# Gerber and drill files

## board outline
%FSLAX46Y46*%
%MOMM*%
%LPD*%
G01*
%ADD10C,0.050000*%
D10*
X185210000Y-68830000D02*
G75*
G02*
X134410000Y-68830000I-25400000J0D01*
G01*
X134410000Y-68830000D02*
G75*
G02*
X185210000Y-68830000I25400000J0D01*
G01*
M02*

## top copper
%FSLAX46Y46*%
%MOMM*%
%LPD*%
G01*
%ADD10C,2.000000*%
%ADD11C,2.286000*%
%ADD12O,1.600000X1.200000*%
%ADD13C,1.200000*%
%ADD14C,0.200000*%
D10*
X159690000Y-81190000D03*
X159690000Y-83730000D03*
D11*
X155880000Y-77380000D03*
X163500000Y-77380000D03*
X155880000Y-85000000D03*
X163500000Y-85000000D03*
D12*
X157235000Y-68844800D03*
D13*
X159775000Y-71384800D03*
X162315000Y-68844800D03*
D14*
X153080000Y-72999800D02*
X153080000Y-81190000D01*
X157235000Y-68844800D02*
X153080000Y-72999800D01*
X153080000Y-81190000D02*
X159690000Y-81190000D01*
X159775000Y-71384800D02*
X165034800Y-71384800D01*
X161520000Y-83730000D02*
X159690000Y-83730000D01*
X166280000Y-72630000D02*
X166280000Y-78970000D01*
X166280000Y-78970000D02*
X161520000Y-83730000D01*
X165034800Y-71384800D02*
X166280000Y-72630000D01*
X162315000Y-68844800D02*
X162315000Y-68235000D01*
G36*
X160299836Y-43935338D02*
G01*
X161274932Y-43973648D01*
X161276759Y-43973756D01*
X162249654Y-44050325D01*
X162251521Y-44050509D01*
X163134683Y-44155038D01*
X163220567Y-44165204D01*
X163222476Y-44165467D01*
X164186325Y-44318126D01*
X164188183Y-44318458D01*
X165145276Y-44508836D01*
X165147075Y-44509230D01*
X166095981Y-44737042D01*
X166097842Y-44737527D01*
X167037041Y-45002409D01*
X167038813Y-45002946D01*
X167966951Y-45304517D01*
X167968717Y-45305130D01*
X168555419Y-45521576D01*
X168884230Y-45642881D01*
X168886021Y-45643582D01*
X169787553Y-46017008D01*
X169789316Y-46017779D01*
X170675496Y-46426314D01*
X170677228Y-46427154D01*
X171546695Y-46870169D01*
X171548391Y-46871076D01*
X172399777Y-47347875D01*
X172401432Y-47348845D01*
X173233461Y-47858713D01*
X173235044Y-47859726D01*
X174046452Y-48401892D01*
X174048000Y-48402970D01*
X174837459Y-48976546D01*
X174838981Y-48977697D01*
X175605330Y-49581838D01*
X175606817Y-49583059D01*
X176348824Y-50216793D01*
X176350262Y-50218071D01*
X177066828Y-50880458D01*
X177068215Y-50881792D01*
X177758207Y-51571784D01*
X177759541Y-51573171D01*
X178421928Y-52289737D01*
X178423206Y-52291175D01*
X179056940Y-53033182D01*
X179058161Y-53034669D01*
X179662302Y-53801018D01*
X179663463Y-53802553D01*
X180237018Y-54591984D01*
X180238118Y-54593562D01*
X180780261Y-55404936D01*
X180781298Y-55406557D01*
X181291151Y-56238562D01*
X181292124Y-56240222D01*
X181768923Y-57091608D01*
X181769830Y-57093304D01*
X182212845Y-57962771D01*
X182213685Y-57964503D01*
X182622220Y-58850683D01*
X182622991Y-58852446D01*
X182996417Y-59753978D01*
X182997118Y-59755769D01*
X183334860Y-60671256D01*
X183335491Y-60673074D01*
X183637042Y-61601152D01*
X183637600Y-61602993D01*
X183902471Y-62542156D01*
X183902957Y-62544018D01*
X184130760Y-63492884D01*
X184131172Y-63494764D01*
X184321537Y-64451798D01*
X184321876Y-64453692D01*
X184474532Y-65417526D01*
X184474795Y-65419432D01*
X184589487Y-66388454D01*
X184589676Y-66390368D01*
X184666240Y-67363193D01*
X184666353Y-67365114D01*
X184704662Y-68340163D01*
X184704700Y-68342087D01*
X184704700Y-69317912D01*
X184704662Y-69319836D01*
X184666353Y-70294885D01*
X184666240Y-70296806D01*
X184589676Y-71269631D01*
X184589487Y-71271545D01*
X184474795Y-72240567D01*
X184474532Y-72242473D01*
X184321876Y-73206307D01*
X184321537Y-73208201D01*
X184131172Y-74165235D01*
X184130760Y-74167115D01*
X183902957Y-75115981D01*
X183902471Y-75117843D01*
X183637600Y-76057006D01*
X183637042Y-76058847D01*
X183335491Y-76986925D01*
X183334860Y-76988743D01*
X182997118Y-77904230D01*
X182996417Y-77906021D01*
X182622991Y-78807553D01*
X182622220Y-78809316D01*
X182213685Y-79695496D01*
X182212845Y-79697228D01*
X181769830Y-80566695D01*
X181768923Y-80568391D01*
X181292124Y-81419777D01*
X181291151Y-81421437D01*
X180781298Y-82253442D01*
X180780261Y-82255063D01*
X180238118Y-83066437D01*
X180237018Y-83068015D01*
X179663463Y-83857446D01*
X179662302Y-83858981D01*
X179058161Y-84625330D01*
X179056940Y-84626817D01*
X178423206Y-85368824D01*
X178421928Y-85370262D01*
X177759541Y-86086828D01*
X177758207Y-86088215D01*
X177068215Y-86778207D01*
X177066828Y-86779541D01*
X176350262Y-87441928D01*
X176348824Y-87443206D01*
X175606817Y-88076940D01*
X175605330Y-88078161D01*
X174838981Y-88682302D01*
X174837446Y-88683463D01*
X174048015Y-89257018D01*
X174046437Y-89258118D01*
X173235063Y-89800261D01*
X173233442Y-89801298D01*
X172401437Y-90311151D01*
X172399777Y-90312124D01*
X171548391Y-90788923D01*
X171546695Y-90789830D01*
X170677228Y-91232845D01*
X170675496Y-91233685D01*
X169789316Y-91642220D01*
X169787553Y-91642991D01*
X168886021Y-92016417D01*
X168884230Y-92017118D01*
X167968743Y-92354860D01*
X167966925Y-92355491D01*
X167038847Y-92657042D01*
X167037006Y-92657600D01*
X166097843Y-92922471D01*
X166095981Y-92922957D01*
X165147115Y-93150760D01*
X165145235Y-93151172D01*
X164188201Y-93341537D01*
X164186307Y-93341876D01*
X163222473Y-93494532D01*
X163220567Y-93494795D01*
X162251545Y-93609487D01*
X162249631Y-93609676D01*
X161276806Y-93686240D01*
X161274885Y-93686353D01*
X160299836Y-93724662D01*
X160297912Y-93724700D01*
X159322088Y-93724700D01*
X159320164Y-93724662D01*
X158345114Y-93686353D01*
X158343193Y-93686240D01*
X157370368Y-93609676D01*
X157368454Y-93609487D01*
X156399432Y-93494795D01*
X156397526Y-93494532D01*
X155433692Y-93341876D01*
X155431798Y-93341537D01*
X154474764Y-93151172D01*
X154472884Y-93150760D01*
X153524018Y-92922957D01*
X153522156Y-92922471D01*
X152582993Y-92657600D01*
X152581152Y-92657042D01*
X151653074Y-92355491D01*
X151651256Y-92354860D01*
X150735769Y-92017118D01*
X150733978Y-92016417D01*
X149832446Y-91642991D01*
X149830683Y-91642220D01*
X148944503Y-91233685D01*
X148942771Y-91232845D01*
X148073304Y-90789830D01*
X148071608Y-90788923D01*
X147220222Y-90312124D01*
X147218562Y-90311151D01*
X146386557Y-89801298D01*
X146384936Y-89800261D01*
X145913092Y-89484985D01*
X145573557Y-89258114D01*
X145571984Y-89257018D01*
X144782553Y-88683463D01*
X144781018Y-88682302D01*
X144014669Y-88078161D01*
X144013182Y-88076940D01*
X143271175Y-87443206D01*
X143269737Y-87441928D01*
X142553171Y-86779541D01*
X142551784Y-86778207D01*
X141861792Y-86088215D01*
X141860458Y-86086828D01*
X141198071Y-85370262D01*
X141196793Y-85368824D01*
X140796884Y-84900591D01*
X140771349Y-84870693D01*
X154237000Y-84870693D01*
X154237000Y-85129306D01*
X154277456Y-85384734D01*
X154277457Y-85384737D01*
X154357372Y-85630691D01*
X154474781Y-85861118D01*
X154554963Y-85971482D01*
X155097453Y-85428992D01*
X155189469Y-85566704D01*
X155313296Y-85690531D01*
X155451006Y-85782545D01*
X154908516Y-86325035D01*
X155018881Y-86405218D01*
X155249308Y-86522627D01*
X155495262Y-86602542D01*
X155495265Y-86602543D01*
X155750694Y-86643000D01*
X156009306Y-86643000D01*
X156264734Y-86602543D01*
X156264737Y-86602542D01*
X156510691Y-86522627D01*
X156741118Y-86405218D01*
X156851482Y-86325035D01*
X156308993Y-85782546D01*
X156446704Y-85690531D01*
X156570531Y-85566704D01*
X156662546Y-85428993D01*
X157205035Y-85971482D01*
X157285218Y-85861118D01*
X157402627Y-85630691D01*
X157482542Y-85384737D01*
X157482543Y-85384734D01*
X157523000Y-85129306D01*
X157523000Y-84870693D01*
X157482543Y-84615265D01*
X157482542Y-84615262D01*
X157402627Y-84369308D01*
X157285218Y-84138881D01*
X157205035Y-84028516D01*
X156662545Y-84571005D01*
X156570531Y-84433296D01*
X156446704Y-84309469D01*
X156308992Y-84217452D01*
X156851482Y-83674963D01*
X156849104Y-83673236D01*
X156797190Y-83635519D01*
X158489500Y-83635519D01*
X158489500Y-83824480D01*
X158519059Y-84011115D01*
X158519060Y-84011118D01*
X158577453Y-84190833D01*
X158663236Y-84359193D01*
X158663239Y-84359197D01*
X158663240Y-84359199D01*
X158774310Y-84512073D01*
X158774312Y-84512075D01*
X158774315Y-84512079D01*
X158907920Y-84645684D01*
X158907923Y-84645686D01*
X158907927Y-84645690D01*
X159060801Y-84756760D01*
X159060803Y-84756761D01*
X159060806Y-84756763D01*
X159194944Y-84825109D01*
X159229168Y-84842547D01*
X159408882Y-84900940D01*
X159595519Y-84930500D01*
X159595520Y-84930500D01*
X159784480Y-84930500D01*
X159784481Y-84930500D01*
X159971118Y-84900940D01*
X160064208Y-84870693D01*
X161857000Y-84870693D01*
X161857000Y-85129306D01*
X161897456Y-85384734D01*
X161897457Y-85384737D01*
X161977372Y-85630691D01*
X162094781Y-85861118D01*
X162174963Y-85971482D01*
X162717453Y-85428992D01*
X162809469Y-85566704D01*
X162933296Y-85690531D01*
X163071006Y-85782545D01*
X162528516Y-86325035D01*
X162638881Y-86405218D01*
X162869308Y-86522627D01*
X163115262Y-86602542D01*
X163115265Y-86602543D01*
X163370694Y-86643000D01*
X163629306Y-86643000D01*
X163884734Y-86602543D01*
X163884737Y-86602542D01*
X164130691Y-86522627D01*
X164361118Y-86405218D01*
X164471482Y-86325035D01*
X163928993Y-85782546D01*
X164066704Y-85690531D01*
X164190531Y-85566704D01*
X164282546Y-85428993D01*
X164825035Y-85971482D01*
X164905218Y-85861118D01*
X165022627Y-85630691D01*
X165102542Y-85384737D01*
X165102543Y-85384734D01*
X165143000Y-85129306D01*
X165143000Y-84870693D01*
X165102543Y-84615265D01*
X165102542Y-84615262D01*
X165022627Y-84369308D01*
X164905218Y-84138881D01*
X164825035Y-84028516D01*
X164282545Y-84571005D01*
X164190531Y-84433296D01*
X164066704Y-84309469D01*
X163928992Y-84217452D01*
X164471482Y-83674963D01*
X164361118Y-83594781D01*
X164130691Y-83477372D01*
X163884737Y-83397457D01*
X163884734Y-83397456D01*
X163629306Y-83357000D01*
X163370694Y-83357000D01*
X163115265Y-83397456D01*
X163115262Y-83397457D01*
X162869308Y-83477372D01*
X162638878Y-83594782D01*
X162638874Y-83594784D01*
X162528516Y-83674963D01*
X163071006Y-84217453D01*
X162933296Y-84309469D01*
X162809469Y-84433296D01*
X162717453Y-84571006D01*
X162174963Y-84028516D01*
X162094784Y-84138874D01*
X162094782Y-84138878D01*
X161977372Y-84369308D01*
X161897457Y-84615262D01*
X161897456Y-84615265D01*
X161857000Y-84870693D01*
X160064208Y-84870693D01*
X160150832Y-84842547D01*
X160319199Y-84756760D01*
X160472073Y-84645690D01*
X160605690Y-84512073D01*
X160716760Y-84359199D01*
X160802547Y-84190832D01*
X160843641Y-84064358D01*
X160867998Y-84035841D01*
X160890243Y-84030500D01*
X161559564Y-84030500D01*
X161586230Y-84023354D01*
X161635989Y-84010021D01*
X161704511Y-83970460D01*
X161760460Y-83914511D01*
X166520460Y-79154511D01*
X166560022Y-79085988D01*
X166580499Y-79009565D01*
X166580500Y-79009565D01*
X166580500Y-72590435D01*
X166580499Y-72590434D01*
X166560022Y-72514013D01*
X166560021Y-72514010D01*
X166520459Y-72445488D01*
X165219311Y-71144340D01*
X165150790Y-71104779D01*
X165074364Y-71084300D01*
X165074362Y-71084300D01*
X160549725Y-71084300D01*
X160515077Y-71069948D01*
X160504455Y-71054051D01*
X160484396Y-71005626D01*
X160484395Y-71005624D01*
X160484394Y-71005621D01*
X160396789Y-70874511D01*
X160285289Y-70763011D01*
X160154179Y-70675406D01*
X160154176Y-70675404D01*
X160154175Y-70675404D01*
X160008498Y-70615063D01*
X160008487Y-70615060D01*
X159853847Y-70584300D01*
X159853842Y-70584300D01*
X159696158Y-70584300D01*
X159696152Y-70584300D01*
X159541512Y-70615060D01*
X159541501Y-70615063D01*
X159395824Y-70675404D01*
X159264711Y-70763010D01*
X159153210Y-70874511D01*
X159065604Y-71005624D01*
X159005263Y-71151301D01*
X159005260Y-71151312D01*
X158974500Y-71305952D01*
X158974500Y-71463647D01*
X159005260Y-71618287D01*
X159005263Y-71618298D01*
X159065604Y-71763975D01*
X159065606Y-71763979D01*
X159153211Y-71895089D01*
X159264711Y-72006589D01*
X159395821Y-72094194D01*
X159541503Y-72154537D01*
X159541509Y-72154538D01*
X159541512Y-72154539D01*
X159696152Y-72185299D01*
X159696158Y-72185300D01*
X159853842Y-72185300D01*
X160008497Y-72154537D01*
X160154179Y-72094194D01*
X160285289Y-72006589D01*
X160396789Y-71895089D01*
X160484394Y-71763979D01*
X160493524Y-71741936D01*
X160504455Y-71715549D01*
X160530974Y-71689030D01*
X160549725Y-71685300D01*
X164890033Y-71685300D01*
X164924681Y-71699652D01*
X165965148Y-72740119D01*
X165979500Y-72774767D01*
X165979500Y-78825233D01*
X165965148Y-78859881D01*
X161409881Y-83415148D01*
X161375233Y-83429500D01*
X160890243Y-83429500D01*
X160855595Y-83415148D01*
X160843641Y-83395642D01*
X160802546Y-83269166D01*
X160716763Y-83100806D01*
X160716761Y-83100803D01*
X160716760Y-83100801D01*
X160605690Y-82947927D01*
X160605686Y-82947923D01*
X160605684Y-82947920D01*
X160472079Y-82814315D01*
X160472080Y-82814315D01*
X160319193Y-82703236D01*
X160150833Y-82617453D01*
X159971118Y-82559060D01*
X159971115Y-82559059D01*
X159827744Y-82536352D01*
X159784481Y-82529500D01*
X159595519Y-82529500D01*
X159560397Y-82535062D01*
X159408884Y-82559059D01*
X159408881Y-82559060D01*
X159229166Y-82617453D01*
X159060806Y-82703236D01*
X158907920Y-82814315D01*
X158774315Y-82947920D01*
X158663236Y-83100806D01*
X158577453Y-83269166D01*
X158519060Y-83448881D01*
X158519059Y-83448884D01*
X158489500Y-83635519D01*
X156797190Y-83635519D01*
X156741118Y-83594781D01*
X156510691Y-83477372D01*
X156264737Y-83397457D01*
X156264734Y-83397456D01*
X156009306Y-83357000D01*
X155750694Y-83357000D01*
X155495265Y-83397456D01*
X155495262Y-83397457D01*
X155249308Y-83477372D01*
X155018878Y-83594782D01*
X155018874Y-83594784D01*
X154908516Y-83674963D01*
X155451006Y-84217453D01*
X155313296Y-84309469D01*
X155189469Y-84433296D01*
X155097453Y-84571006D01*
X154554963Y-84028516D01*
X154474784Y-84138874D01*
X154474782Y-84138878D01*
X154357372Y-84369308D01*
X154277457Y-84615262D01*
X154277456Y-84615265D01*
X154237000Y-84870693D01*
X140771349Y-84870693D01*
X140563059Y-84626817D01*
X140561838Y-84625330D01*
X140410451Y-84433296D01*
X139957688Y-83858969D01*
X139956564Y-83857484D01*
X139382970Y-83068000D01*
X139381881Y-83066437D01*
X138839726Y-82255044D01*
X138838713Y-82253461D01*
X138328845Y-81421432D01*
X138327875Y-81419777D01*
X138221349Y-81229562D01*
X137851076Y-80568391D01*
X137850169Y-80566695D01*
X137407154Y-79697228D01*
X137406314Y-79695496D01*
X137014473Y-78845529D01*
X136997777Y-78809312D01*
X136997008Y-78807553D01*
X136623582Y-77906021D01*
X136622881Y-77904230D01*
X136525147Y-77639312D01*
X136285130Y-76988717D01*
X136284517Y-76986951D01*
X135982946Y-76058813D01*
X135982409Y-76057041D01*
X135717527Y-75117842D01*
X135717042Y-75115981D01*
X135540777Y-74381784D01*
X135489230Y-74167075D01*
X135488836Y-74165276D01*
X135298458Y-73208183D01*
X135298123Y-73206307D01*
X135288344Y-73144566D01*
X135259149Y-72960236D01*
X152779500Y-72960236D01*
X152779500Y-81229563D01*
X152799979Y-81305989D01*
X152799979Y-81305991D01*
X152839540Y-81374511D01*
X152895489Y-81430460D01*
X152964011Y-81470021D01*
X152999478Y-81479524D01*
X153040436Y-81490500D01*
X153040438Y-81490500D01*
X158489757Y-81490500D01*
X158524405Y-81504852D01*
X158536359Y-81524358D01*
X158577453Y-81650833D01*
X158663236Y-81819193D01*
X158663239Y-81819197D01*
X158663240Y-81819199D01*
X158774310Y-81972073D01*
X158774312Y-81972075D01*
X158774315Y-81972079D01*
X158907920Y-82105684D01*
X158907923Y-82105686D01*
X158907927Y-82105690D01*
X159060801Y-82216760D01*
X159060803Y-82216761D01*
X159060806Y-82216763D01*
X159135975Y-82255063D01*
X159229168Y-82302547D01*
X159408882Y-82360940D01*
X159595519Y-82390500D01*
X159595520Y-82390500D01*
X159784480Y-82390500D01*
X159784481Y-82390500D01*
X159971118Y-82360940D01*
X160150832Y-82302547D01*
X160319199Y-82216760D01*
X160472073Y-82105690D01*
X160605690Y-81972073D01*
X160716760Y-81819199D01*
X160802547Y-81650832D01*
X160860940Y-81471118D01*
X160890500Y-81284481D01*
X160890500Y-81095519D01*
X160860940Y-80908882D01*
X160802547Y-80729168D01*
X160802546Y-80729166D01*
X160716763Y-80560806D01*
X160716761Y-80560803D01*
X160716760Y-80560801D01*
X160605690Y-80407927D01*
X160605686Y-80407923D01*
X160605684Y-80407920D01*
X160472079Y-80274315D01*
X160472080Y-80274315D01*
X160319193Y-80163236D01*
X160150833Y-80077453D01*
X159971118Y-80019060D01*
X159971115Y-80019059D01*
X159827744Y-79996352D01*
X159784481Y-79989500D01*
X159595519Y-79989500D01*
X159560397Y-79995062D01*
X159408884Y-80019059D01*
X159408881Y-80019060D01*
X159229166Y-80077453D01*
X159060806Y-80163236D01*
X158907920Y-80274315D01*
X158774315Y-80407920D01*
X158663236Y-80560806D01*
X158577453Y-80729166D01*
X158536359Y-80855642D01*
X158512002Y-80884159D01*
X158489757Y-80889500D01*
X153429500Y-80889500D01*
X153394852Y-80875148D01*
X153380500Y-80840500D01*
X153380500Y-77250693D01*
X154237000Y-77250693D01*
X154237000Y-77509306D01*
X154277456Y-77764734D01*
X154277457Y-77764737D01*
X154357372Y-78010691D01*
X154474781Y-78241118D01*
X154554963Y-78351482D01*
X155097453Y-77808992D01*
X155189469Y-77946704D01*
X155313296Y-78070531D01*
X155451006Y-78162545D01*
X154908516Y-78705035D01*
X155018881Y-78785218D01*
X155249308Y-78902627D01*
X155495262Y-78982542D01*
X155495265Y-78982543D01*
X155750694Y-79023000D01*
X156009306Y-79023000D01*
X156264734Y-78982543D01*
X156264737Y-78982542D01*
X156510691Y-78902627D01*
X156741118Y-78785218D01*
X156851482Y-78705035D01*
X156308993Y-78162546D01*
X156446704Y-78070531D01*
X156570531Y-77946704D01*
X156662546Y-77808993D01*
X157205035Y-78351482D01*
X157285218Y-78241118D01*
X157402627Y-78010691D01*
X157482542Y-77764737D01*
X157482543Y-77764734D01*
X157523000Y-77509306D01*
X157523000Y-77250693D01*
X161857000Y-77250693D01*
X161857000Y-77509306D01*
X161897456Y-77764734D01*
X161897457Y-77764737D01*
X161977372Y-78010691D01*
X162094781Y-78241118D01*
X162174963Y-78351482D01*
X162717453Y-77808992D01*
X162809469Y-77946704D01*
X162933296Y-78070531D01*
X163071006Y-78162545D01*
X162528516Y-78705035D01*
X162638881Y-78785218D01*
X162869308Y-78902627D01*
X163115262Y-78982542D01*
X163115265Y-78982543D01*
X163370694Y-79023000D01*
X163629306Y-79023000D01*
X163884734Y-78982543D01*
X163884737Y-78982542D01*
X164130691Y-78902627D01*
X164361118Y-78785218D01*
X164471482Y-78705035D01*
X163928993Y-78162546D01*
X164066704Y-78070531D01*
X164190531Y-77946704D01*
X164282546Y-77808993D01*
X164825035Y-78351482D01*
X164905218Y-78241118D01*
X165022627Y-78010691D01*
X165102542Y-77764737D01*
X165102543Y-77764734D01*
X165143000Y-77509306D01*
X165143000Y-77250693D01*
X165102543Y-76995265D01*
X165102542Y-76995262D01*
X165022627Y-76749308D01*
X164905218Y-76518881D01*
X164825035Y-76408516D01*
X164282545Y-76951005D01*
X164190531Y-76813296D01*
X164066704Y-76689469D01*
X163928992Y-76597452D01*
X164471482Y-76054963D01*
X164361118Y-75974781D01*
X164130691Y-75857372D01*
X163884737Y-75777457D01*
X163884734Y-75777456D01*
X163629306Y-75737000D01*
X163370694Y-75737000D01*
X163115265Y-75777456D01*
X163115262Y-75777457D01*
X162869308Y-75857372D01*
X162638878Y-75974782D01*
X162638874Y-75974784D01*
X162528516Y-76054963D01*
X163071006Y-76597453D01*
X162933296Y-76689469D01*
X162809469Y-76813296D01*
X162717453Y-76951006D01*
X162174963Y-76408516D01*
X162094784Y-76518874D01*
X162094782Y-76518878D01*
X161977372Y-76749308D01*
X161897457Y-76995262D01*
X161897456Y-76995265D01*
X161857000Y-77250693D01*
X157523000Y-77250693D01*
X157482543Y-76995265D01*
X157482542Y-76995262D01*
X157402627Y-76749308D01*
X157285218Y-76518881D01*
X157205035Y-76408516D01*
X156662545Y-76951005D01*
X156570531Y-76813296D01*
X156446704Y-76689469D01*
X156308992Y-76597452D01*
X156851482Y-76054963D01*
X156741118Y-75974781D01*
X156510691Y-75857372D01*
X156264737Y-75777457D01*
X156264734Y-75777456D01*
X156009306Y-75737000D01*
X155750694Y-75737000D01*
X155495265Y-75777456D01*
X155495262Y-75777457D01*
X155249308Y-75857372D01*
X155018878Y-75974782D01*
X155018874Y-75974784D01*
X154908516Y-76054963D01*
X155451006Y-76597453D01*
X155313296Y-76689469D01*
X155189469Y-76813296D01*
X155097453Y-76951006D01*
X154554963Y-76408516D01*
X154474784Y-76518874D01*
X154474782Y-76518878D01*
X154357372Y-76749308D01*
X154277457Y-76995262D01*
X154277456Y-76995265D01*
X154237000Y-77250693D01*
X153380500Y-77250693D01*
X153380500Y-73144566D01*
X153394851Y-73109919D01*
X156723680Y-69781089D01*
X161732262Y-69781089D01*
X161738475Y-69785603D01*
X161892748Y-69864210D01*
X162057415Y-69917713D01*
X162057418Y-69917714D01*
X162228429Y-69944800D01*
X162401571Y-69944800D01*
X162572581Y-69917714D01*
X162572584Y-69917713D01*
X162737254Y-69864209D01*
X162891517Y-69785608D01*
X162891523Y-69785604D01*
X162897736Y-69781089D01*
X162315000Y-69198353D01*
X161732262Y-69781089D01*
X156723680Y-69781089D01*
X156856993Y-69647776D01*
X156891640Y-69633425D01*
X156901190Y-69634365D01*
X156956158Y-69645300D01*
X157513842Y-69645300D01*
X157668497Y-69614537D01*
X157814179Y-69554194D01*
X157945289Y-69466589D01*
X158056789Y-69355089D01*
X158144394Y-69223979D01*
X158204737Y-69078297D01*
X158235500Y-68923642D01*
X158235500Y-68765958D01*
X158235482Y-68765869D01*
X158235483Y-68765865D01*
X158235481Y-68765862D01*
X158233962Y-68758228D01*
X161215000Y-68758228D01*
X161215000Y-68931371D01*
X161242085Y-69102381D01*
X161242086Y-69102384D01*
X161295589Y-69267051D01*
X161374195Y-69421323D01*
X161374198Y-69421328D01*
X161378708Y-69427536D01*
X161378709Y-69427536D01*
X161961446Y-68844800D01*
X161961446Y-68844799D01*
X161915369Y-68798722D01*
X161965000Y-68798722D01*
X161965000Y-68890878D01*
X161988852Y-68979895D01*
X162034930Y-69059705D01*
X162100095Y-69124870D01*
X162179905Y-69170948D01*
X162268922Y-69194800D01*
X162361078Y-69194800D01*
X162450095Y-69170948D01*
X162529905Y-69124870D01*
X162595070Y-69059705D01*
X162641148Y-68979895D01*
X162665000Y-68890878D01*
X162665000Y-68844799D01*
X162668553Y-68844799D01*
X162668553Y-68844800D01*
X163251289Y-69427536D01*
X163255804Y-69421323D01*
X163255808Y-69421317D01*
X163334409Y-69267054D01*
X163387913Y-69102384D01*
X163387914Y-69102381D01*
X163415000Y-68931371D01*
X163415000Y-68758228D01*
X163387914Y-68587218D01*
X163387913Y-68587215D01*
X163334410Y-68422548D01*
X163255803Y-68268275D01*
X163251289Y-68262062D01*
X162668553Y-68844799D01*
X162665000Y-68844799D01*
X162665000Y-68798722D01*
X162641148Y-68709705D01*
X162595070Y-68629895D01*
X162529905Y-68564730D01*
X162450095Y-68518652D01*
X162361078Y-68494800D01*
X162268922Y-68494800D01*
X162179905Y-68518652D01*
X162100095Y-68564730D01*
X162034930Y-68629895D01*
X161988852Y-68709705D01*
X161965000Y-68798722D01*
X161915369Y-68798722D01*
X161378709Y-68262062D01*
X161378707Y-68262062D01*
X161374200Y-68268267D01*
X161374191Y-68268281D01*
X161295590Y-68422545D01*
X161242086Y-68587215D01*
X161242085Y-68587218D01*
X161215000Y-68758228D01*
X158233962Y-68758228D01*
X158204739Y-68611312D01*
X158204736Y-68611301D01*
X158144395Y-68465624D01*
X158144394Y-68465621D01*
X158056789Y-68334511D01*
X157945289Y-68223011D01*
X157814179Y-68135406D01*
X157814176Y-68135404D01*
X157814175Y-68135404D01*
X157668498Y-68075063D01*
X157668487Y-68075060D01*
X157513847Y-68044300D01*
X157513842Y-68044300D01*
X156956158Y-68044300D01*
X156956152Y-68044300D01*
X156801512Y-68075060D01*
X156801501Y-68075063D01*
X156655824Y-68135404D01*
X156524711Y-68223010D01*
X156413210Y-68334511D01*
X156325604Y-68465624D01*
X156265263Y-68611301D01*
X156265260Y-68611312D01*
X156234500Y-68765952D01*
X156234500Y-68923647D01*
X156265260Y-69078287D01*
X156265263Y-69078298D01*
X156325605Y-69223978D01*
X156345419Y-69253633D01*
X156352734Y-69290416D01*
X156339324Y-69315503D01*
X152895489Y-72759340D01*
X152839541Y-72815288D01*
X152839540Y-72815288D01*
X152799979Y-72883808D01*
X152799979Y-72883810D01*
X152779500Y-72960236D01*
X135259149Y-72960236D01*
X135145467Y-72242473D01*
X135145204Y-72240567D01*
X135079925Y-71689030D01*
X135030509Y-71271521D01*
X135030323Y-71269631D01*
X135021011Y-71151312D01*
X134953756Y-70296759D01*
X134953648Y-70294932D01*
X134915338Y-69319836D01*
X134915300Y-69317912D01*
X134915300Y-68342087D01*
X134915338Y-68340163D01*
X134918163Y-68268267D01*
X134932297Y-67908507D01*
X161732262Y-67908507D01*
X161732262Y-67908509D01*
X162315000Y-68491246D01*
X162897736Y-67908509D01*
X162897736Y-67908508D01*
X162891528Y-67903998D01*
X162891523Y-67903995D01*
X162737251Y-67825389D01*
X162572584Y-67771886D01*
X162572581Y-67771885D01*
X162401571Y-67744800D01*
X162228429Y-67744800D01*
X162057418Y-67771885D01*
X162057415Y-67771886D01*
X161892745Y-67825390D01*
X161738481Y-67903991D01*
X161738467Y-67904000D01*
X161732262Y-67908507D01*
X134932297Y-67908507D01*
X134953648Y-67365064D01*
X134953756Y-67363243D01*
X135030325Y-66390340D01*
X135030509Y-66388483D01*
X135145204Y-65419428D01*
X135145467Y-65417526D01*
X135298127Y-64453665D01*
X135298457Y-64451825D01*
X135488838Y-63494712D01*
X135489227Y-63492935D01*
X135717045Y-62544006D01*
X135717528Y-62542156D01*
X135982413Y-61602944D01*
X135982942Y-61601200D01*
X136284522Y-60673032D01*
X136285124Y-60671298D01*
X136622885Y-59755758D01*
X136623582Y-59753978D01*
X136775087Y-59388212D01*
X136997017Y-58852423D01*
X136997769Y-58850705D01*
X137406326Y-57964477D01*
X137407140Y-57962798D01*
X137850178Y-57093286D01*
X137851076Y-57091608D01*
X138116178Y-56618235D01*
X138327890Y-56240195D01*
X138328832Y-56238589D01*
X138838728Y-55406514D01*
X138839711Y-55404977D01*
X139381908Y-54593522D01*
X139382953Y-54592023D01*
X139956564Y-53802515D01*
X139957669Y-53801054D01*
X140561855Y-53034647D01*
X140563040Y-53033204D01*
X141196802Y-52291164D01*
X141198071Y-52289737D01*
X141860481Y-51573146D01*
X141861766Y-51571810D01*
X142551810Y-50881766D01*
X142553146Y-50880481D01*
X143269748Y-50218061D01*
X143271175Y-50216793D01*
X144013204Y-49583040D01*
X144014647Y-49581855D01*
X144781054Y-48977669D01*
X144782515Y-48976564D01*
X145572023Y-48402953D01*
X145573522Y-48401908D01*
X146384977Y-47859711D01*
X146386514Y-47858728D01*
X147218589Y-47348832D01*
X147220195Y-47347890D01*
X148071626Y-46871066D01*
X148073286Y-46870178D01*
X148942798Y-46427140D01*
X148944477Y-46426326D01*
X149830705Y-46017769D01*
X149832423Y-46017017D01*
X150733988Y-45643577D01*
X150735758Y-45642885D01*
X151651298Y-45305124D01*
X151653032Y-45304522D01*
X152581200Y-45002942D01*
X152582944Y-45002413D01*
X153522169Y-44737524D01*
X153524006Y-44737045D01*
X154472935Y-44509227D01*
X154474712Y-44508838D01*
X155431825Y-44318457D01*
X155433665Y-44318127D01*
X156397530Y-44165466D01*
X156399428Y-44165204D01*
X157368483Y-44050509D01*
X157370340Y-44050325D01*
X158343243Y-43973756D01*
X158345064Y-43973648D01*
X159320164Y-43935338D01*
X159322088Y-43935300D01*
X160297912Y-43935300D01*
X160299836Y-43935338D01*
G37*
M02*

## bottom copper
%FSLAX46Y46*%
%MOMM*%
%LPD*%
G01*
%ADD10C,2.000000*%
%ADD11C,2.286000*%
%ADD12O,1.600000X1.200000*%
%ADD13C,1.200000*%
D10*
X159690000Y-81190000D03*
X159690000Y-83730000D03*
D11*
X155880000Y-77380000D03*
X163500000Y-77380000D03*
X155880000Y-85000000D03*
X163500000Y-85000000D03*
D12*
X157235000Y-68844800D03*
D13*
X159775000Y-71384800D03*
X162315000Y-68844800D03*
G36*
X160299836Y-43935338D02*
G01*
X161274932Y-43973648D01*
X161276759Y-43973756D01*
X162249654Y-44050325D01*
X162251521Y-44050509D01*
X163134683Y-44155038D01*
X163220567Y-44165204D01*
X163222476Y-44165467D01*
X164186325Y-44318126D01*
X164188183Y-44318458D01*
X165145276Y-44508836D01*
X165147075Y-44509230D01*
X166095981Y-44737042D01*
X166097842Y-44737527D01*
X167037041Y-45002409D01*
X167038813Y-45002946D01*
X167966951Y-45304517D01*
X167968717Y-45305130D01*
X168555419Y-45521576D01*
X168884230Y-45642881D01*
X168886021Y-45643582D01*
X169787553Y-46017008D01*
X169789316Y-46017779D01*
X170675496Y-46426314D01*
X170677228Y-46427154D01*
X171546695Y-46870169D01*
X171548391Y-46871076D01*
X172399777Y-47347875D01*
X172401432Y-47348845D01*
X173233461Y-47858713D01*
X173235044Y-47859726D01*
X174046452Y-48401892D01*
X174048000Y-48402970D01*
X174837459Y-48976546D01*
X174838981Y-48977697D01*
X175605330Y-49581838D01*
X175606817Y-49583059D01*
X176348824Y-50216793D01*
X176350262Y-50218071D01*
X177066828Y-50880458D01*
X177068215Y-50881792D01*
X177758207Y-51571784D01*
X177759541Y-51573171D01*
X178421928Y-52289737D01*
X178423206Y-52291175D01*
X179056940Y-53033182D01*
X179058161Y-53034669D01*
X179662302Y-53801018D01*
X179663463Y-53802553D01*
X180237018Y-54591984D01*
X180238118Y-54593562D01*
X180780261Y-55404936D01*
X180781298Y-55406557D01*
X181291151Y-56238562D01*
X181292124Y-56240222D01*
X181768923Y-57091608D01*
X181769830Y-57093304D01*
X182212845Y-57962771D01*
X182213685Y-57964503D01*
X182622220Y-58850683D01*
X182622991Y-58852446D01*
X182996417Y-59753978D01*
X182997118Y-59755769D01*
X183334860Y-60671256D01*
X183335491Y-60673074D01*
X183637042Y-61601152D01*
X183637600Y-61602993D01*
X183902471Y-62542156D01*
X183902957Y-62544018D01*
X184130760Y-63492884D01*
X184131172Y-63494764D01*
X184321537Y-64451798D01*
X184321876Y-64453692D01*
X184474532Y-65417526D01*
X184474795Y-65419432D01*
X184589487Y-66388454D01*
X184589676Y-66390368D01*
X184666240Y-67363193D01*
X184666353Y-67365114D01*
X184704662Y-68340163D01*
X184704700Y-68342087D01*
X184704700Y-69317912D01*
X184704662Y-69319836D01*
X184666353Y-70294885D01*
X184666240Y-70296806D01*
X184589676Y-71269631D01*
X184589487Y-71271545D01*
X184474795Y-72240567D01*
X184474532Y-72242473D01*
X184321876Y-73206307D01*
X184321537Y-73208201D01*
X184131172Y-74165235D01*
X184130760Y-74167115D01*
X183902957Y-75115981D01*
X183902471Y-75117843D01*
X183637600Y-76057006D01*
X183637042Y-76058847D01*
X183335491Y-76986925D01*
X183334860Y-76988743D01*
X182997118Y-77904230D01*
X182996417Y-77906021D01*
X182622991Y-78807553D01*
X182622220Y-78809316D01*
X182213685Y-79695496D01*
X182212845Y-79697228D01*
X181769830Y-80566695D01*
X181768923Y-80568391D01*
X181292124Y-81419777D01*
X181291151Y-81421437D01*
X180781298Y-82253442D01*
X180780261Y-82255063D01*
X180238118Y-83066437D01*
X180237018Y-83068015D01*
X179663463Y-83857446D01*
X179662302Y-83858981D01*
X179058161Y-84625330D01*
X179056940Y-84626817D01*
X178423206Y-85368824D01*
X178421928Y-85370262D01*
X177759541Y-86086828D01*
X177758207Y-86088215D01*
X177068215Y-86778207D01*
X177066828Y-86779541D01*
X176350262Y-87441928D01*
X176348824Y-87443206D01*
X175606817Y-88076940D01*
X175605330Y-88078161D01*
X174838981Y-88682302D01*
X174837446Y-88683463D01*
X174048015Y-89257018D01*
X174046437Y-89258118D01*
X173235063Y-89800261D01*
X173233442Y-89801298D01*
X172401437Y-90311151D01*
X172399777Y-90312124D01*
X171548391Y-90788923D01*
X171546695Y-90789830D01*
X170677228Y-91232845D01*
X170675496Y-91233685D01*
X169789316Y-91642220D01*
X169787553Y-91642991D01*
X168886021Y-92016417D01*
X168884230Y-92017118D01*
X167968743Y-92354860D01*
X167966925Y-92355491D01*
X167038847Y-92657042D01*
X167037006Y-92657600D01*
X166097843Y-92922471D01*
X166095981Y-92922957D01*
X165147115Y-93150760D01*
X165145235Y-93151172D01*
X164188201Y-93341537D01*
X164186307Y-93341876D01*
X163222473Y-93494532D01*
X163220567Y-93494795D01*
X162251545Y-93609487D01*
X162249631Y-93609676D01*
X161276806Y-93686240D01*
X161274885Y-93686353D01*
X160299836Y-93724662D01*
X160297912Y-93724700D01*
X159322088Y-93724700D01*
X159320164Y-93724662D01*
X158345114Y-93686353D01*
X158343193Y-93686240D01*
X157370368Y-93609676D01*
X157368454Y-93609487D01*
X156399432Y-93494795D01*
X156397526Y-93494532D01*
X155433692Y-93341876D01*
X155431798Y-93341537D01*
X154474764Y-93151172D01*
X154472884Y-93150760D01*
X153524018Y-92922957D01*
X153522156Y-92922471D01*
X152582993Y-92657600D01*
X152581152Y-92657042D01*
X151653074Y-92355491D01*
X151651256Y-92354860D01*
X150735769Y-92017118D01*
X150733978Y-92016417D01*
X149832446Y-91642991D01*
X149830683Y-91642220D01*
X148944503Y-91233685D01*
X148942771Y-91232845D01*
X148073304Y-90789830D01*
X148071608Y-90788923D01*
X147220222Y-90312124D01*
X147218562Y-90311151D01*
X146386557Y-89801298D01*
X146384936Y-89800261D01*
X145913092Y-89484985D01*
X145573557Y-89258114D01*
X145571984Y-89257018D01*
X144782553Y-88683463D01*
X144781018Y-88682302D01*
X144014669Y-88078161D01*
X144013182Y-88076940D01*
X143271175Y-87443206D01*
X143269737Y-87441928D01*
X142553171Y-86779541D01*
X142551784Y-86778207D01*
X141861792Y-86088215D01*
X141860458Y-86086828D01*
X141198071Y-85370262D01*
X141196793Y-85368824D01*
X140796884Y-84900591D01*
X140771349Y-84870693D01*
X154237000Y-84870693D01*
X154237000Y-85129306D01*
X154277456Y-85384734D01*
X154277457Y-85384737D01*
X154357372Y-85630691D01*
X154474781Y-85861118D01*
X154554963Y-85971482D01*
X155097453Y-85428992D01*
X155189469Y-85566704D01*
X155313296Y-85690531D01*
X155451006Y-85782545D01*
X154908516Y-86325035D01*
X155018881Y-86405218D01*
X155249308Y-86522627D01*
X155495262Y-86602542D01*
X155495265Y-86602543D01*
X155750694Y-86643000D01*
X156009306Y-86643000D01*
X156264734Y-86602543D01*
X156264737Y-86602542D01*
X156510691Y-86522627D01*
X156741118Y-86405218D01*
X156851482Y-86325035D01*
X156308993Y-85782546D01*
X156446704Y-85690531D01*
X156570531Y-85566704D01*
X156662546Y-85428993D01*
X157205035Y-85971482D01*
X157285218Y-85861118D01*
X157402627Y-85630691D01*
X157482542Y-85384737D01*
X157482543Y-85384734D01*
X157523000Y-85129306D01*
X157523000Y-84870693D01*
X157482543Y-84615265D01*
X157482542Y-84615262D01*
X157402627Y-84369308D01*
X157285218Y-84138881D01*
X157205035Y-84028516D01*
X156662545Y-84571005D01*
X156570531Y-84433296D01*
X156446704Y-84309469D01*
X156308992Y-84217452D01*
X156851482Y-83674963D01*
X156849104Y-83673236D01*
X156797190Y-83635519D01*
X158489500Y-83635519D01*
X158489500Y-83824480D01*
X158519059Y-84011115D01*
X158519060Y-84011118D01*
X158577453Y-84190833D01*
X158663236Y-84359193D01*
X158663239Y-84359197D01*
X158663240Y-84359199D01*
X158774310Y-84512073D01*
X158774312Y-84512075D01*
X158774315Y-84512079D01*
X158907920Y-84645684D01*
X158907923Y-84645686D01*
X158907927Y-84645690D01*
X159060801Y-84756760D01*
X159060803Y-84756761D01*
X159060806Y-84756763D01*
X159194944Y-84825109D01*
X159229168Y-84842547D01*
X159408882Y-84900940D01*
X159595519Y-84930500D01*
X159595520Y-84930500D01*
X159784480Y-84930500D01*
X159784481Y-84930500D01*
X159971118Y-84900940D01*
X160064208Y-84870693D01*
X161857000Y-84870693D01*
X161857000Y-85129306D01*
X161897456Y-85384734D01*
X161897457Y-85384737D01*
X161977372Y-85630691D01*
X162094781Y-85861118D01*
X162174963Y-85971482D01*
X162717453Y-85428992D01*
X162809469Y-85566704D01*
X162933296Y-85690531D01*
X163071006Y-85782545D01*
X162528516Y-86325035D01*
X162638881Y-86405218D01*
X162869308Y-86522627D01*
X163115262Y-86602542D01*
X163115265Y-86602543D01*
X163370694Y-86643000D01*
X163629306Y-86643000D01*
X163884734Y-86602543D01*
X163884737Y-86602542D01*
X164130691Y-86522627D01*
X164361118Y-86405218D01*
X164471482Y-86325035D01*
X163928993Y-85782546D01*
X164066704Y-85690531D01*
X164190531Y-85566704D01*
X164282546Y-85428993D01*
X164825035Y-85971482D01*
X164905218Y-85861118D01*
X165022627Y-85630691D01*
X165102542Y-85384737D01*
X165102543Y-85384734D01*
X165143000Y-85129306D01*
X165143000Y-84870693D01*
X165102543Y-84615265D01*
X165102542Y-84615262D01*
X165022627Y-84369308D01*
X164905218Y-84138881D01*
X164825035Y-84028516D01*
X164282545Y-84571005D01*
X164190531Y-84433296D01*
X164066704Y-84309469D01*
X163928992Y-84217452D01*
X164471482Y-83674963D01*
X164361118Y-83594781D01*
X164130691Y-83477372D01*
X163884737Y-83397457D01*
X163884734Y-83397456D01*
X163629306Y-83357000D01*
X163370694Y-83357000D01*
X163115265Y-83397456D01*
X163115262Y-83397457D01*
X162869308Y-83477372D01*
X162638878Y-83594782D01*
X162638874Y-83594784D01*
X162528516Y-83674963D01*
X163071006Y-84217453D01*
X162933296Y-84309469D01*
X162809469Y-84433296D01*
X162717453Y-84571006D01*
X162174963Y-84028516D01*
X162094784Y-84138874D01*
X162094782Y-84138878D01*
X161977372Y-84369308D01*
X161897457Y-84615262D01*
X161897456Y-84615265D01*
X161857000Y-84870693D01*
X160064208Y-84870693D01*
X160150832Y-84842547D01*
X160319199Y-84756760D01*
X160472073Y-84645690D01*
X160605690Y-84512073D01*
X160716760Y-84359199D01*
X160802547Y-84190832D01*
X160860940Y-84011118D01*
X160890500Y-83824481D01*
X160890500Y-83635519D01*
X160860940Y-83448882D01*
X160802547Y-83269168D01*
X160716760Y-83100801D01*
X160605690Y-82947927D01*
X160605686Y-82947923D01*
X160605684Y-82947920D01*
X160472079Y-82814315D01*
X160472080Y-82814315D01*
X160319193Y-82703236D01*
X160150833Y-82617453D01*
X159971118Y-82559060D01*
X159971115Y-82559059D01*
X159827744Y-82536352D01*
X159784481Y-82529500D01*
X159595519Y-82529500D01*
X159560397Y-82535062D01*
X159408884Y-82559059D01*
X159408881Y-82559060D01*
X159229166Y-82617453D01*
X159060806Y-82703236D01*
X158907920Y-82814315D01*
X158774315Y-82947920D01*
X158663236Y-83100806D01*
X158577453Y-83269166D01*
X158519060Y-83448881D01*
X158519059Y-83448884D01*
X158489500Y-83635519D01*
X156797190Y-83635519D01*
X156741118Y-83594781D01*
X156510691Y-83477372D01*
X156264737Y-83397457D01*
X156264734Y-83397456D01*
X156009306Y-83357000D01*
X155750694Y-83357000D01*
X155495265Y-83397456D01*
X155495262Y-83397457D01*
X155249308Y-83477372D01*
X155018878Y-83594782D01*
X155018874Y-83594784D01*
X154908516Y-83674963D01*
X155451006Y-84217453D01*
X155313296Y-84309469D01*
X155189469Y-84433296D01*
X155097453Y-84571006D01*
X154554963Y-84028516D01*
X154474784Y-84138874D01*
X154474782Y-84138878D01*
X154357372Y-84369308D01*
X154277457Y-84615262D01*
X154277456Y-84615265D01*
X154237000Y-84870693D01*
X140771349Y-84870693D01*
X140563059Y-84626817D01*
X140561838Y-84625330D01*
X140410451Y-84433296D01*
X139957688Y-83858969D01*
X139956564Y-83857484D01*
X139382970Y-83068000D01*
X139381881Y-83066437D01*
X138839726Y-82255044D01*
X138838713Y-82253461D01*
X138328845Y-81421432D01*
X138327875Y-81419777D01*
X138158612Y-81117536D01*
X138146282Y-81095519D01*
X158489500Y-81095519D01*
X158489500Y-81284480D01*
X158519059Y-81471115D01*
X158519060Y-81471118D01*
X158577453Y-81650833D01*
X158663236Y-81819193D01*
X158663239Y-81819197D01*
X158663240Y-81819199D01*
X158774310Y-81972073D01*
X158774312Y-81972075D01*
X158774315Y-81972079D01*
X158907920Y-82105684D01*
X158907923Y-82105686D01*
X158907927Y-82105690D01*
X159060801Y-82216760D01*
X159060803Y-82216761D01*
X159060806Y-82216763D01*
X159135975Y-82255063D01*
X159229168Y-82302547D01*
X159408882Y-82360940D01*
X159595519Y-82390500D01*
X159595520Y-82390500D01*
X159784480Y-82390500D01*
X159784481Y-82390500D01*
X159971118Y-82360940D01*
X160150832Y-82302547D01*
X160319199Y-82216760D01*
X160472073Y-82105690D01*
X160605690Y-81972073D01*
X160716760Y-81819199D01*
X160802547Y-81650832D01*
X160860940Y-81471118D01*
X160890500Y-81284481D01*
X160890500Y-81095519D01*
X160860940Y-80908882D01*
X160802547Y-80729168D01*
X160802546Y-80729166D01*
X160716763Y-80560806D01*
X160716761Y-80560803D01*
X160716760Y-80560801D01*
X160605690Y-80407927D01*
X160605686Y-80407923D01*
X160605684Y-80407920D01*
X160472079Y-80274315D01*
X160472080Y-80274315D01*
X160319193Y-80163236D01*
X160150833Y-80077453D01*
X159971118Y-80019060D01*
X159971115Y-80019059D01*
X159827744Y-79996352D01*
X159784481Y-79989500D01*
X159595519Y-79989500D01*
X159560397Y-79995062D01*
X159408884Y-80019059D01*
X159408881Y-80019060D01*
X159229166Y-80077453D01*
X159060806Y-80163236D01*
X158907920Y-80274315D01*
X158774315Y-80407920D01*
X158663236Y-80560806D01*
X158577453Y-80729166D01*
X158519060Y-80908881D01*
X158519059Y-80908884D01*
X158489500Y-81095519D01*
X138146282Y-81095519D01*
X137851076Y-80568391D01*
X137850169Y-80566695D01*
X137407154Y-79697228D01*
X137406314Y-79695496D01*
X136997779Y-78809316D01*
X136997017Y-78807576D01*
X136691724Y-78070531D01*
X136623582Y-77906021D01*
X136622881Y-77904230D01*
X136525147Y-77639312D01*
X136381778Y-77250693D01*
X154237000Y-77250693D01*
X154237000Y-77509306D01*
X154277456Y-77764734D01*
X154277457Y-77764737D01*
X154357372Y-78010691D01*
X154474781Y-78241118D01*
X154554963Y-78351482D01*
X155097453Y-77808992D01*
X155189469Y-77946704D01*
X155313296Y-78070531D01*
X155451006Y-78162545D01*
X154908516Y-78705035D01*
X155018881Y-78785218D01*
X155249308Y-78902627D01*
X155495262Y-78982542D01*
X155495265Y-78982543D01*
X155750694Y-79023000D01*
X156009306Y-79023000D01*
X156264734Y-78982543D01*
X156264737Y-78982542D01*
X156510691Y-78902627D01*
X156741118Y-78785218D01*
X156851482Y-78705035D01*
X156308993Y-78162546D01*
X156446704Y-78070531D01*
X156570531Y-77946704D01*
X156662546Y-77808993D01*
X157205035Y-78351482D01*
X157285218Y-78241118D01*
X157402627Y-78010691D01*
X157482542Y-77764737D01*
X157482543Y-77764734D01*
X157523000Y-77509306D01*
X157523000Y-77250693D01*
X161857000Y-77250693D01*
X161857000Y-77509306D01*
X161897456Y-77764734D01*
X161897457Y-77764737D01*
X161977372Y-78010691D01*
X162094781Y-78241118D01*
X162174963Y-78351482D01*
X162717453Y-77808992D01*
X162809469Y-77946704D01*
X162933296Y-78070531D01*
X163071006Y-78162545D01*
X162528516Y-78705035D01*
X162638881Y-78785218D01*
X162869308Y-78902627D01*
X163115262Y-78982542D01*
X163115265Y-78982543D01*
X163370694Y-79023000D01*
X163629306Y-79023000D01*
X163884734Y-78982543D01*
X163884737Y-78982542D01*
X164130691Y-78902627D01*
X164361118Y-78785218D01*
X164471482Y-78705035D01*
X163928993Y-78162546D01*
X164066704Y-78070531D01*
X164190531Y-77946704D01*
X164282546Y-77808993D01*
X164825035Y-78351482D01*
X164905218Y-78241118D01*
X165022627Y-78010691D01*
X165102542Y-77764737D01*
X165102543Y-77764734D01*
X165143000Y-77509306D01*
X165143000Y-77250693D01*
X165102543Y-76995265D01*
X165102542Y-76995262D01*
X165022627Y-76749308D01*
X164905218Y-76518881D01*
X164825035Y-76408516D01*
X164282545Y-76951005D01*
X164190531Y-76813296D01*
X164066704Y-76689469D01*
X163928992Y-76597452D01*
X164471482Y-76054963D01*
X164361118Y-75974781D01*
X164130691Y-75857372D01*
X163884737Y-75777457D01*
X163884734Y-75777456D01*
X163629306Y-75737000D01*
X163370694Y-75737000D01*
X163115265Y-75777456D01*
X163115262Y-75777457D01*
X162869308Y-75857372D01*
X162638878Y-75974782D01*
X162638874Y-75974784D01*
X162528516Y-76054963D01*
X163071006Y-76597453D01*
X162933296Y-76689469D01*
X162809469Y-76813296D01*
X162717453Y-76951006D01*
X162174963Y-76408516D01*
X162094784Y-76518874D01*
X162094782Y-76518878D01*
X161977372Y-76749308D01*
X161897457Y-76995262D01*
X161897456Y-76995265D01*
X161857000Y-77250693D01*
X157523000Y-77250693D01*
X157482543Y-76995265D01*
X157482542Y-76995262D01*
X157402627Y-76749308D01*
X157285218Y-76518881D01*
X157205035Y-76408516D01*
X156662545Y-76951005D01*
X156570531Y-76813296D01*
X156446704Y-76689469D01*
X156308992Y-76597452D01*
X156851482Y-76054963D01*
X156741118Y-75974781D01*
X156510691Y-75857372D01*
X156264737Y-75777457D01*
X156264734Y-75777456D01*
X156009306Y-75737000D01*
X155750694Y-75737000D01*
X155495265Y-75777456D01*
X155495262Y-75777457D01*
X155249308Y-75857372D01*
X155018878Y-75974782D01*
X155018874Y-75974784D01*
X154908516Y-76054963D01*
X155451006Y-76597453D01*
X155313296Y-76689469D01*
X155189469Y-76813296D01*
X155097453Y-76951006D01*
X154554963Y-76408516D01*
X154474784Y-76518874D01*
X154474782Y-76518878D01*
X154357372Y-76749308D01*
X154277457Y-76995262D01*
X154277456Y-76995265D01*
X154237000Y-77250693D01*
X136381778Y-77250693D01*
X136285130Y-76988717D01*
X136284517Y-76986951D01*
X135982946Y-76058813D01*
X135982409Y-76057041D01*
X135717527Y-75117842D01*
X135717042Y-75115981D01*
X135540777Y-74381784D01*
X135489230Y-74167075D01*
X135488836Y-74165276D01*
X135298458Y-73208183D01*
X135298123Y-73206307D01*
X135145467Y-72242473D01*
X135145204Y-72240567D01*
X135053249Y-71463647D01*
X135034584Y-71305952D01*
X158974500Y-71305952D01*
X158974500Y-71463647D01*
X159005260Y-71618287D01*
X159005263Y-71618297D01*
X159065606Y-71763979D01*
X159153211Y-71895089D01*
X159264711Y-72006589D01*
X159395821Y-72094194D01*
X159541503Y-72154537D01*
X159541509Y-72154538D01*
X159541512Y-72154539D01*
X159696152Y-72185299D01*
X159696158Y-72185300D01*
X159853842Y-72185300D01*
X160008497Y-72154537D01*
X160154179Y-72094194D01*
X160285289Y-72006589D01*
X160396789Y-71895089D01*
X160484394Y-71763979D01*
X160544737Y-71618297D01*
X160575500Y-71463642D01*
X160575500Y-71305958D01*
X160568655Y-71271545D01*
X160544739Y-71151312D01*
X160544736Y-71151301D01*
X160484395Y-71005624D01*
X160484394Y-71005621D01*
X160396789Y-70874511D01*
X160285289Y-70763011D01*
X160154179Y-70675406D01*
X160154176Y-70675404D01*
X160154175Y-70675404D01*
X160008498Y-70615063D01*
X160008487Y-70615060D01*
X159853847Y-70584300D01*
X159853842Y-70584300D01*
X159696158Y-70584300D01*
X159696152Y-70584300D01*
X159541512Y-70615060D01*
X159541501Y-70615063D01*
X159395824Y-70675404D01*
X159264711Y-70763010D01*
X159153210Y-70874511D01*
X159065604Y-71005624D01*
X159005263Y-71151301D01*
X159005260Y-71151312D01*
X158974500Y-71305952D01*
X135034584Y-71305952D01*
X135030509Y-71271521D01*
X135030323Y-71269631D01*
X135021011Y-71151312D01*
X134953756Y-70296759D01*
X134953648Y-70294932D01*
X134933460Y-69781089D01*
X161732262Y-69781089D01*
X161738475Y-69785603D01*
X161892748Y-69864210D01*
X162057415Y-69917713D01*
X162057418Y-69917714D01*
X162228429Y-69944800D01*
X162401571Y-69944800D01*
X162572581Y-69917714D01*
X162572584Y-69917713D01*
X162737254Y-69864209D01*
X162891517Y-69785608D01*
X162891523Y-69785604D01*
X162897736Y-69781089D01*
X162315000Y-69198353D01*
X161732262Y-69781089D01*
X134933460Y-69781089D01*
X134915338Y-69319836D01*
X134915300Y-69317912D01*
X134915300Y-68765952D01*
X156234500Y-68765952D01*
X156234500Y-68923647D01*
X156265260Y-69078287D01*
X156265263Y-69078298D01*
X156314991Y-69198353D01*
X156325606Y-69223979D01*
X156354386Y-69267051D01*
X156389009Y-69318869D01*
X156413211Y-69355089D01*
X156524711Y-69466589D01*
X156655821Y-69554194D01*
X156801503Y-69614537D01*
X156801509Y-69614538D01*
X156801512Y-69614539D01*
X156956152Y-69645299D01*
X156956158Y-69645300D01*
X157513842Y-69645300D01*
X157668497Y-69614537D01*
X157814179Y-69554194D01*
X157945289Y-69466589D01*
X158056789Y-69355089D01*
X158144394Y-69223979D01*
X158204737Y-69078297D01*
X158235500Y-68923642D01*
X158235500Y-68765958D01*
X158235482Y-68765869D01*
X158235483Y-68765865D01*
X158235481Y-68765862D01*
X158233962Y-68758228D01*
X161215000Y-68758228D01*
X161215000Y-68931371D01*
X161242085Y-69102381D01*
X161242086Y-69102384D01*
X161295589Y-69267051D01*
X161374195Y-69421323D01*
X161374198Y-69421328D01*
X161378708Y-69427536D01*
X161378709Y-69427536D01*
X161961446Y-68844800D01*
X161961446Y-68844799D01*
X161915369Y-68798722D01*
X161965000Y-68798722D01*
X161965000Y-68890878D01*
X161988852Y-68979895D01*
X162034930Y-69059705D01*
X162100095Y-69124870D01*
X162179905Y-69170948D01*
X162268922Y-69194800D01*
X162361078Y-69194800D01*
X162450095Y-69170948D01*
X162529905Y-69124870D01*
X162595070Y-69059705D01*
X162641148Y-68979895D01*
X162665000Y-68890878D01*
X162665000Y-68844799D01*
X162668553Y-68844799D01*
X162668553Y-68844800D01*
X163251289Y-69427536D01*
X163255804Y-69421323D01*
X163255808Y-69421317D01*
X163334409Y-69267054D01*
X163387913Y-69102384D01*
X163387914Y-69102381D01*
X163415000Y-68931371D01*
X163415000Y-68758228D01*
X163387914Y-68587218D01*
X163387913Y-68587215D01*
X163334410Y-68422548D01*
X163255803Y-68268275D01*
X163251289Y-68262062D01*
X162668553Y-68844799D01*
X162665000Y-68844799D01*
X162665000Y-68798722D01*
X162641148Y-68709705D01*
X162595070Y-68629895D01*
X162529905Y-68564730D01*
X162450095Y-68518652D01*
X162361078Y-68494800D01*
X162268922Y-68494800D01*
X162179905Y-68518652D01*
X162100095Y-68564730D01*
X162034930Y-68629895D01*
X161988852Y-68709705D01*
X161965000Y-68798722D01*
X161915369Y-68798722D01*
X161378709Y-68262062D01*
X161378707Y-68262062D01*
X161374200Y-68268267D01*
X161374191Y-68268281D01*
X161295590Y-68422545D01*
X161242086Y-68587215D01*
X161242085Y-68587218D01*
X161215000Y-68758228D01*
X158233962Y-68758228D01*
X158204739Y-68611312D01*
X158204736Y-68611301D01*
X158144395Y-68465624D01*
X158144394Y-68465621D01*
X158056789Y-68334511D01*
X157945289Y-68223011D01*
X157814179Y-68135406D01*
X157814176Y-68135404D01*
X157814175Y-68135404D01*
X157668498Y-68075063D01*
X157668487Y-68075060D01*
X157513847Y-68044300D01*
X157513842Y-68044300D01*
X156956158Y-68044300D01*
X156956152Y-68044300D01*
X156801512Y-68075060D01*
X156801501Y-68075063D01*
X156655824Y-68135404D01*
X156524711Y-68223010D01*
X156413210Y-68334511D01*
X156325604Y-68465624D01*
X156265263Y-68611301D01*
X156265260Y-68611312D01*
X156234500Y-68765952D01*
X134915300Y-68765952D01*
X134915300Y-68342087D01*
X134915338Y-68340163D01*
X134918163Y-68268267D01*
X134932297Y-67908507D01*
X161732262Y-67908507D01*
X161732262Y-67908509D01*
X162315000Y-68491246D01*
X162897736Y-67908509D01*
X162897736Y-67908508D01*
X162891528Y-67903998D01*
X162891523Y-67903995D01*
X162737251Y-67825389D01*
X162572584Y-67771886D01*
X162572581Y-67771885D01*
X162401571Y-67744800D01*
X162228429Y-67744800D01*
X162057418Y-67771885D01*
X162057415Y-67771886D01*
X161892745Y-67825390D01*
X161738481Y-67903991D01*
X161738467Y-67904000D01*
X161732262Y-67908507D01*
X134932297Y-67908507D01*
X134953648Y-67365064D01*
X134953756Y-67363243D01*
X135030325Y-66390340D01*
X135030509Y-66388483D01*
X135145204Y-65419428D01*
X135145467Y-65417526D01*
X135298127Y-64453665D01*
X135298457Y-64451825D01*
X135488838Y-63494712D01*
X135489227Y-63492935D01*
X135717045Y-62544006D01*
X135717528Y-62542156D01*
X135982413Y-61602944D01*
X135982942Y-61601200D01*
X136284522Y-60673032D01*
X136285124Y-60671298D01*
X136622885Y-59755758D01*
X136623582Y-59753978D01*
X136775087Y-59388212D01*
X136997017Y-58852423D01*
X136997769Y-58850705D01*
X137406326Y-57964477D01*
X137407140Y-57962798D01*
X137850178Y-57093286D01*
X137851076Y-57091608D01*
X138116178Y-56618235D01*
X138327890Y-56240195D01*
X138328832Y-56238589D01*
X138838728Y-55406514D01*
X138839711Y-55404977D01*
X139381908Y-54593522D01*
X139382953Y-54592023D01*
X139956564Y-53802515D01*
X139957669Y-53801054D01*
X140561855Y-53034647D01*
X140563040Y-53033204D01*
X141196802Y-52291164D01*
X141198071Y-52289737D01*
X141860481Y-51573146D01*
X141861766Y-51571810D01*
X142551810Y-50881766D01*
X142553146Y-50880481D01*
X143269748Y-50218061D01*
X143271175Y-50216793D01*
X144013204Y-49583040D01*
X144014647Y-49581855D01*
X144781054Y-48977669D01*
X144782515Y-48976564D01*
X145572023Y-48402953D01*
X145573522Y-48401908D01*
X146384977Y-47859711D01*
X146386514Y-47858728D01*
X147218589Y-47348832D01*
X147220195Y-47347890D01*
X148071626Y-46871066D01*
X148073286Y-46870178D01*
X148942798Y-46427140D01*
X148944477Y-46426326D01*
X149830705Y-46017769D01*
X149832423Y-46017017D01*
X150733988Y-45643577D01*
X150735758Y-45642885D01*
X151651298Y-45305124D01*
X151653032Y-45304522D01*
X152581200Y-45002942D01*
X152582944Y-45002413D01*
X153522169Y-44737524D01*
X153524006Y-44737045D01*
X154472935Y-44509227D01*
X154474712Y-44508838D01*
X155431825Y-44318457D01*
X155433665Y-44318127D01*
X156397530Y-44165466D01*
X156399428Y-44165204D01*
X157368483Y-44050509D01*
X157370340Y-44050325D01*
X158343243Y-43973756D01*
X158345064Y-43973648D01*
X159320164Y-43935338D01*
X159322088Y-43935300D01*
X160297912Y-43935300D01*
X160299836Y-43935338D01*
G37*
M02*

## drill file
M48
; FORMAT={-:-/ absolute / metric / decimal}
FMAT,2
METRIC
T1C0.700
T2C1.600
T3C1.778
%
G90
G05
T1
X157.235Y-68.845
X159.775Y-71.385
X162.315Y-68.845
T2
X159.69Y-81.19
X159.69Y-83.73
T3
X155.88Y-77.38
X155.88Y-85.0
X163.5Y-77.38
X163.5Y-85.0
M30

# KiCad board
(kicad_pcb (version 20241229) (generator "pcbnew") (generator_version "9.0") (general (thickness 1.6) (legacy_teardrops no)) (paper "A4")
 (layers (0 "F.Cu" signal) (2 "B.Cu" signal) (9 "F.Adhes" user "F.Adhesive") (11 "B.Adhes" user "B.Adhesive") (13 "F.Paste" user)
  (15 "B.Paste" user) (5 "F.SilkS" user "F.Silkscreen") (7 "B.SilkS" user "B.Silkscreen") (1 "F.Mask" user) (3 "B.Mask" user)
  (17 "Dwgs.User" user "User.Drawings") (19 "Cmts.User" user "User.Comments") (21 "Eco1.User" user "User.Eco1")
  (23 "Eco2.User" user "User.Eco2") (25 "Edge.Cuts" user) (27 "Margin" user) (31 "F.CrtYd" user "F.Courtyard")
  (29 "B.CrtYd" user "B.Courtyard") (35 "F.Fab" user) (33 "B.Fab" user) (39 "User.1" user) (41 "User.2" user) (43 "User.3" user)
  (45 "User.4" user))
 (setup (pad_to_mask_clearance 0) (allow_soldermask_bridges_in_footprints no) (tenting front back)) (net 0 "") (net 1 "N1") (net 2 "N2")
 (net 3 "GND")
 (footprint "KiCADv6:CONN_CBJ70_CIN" (layer "F.Cu") (at 159.69 81.19)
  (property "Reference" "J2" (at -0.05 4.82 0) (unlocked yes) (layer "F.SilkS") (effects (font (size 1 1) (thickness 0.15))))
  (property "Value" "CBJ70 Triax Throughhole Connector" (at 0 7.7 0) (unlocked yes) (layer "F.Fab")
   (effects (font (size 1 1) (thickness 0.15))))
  (pad "1" thru_hole circle (at 0 0) (size 2 2) (drill 1.6) (layers "*.Cu" "*.Mask") (remove_unused_layers no) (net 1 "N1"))
  (pad "2" thru_hole circle (at 0 2.54) (size 2 2) (drill 1.6) (layers "*.Cu" "*.Mask") (remove_unused_layers no) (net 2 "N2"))
  (pad "3" thru_hole circle (at -3.81 -3.81) (size 2.286 2.286) (drill 1.778) (layers "*.Cu" "*.Mask") (remove_unused_layers no)
   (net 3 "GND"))
  (pad "4" thru_hole circle (at 3.81 -3.81) (size 2.286 2.286) (drill 1.778) (layers "*.Cu" "*.Mask") (remove_unused_layers no)
   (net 3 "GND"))
  (pad "5" thru_hole circle (at -3.81 3.81) (size 2.286 2.286) (drill 1.778) (layers "*.Cu" "*.Mask") (remove_unused_layers no)
   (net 3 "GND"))
  (pad "6" thru_hole circle (at 3.81 3.81) (size 2.286 2.286) (drill 1.778) (layers "*.Cu" "*.Mask") (remove_unused_layers no) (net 3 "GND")))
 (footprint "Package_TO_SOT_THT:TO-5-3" (layer "F.Cu") (at 157.235 68.8448)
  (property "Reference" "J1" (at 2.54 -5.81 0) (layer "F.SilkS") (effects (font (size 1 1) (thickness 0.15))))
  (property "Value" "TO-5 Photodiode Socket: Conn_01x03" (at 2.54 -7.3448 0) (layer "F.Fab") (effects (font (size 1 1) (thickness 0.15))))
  (pad "1" thru_hole oval (at 0 0) (size 1.6 1.2) (drill 0.7) (layers "*.Cu" "*.Mask") (remove_unused_layers no) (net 1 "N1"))
  (pad "2" thru_hole circle (at 2.54 2.54) (size 1.2 1.2) (drill 0.7) (layers "*.Cu" "*.Mask") (remove_unused_layers no) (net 2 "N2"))
  (pad "3" thru_hole circle (at 5.08 0) (size 1.2 1.2) (drill 0.7) (layers "*.Cu" "*.Mask") (remove_unused_layers no) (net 3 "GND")))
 (gr_circle (center 159.81 68.83) (end 185.21 68.83) (stroke (width 0.05) (type solid)) (fill no) (layer "Edge.Cuts"))
 (segment (start 153.08 72.9998) (end 153.08 81.19) (width 0.2) (layer "F.Cu") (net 1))
 (segment (start 157.235 68.8448) (end 153.08 72.9998) (width 0.2) (layer "F.Cu") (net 1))
 (segment (start 153.08 81.19) (end 159.69 81.19) (width 0.2) (layer "F.Cu") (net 1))
 (segment (start 159.775 71.3848) (end 165.0348 71.3848) (width 0.2) (layer "F.Cu") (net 2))
 (segment (start 161.52 83.73) (end 159.69 83.73) (width 0.2) (layer "F.Cu") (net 2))
 (segment (start 166.28 72.63) (end 166.28 78.97) (width 0.2) (layer "F.Cu") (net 2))
 (segment (start 166.28 78.97) (end 161.52 83.73) (width 0.2) (layer "F.Cu") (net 2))
 (segment (start 165.0348 71.3848) (end 166.28 72.63) (width 0.2) (layer "F.Cu") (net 2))
 (segment (start 162.315 68.8448) (end 162.315 68.235) (width 0.2) (layer "F.Cu") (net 3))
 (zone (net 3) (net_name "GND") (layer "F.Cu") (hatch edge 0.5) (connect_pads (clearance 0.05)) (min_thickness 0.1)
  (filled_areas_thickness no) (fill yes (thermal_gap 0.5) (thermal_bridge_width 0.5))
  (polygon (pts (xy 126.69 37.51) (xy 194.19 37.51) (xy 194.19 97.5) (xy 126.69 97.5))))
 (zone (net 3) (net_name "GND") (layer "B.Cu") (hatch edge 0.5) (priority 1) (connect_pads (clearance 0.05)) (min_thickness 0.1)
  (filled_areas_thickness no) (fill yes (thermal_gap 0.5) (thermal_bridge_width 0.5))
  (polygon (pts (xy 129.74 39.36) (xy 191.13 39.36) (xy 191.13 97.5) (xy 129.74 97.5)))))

